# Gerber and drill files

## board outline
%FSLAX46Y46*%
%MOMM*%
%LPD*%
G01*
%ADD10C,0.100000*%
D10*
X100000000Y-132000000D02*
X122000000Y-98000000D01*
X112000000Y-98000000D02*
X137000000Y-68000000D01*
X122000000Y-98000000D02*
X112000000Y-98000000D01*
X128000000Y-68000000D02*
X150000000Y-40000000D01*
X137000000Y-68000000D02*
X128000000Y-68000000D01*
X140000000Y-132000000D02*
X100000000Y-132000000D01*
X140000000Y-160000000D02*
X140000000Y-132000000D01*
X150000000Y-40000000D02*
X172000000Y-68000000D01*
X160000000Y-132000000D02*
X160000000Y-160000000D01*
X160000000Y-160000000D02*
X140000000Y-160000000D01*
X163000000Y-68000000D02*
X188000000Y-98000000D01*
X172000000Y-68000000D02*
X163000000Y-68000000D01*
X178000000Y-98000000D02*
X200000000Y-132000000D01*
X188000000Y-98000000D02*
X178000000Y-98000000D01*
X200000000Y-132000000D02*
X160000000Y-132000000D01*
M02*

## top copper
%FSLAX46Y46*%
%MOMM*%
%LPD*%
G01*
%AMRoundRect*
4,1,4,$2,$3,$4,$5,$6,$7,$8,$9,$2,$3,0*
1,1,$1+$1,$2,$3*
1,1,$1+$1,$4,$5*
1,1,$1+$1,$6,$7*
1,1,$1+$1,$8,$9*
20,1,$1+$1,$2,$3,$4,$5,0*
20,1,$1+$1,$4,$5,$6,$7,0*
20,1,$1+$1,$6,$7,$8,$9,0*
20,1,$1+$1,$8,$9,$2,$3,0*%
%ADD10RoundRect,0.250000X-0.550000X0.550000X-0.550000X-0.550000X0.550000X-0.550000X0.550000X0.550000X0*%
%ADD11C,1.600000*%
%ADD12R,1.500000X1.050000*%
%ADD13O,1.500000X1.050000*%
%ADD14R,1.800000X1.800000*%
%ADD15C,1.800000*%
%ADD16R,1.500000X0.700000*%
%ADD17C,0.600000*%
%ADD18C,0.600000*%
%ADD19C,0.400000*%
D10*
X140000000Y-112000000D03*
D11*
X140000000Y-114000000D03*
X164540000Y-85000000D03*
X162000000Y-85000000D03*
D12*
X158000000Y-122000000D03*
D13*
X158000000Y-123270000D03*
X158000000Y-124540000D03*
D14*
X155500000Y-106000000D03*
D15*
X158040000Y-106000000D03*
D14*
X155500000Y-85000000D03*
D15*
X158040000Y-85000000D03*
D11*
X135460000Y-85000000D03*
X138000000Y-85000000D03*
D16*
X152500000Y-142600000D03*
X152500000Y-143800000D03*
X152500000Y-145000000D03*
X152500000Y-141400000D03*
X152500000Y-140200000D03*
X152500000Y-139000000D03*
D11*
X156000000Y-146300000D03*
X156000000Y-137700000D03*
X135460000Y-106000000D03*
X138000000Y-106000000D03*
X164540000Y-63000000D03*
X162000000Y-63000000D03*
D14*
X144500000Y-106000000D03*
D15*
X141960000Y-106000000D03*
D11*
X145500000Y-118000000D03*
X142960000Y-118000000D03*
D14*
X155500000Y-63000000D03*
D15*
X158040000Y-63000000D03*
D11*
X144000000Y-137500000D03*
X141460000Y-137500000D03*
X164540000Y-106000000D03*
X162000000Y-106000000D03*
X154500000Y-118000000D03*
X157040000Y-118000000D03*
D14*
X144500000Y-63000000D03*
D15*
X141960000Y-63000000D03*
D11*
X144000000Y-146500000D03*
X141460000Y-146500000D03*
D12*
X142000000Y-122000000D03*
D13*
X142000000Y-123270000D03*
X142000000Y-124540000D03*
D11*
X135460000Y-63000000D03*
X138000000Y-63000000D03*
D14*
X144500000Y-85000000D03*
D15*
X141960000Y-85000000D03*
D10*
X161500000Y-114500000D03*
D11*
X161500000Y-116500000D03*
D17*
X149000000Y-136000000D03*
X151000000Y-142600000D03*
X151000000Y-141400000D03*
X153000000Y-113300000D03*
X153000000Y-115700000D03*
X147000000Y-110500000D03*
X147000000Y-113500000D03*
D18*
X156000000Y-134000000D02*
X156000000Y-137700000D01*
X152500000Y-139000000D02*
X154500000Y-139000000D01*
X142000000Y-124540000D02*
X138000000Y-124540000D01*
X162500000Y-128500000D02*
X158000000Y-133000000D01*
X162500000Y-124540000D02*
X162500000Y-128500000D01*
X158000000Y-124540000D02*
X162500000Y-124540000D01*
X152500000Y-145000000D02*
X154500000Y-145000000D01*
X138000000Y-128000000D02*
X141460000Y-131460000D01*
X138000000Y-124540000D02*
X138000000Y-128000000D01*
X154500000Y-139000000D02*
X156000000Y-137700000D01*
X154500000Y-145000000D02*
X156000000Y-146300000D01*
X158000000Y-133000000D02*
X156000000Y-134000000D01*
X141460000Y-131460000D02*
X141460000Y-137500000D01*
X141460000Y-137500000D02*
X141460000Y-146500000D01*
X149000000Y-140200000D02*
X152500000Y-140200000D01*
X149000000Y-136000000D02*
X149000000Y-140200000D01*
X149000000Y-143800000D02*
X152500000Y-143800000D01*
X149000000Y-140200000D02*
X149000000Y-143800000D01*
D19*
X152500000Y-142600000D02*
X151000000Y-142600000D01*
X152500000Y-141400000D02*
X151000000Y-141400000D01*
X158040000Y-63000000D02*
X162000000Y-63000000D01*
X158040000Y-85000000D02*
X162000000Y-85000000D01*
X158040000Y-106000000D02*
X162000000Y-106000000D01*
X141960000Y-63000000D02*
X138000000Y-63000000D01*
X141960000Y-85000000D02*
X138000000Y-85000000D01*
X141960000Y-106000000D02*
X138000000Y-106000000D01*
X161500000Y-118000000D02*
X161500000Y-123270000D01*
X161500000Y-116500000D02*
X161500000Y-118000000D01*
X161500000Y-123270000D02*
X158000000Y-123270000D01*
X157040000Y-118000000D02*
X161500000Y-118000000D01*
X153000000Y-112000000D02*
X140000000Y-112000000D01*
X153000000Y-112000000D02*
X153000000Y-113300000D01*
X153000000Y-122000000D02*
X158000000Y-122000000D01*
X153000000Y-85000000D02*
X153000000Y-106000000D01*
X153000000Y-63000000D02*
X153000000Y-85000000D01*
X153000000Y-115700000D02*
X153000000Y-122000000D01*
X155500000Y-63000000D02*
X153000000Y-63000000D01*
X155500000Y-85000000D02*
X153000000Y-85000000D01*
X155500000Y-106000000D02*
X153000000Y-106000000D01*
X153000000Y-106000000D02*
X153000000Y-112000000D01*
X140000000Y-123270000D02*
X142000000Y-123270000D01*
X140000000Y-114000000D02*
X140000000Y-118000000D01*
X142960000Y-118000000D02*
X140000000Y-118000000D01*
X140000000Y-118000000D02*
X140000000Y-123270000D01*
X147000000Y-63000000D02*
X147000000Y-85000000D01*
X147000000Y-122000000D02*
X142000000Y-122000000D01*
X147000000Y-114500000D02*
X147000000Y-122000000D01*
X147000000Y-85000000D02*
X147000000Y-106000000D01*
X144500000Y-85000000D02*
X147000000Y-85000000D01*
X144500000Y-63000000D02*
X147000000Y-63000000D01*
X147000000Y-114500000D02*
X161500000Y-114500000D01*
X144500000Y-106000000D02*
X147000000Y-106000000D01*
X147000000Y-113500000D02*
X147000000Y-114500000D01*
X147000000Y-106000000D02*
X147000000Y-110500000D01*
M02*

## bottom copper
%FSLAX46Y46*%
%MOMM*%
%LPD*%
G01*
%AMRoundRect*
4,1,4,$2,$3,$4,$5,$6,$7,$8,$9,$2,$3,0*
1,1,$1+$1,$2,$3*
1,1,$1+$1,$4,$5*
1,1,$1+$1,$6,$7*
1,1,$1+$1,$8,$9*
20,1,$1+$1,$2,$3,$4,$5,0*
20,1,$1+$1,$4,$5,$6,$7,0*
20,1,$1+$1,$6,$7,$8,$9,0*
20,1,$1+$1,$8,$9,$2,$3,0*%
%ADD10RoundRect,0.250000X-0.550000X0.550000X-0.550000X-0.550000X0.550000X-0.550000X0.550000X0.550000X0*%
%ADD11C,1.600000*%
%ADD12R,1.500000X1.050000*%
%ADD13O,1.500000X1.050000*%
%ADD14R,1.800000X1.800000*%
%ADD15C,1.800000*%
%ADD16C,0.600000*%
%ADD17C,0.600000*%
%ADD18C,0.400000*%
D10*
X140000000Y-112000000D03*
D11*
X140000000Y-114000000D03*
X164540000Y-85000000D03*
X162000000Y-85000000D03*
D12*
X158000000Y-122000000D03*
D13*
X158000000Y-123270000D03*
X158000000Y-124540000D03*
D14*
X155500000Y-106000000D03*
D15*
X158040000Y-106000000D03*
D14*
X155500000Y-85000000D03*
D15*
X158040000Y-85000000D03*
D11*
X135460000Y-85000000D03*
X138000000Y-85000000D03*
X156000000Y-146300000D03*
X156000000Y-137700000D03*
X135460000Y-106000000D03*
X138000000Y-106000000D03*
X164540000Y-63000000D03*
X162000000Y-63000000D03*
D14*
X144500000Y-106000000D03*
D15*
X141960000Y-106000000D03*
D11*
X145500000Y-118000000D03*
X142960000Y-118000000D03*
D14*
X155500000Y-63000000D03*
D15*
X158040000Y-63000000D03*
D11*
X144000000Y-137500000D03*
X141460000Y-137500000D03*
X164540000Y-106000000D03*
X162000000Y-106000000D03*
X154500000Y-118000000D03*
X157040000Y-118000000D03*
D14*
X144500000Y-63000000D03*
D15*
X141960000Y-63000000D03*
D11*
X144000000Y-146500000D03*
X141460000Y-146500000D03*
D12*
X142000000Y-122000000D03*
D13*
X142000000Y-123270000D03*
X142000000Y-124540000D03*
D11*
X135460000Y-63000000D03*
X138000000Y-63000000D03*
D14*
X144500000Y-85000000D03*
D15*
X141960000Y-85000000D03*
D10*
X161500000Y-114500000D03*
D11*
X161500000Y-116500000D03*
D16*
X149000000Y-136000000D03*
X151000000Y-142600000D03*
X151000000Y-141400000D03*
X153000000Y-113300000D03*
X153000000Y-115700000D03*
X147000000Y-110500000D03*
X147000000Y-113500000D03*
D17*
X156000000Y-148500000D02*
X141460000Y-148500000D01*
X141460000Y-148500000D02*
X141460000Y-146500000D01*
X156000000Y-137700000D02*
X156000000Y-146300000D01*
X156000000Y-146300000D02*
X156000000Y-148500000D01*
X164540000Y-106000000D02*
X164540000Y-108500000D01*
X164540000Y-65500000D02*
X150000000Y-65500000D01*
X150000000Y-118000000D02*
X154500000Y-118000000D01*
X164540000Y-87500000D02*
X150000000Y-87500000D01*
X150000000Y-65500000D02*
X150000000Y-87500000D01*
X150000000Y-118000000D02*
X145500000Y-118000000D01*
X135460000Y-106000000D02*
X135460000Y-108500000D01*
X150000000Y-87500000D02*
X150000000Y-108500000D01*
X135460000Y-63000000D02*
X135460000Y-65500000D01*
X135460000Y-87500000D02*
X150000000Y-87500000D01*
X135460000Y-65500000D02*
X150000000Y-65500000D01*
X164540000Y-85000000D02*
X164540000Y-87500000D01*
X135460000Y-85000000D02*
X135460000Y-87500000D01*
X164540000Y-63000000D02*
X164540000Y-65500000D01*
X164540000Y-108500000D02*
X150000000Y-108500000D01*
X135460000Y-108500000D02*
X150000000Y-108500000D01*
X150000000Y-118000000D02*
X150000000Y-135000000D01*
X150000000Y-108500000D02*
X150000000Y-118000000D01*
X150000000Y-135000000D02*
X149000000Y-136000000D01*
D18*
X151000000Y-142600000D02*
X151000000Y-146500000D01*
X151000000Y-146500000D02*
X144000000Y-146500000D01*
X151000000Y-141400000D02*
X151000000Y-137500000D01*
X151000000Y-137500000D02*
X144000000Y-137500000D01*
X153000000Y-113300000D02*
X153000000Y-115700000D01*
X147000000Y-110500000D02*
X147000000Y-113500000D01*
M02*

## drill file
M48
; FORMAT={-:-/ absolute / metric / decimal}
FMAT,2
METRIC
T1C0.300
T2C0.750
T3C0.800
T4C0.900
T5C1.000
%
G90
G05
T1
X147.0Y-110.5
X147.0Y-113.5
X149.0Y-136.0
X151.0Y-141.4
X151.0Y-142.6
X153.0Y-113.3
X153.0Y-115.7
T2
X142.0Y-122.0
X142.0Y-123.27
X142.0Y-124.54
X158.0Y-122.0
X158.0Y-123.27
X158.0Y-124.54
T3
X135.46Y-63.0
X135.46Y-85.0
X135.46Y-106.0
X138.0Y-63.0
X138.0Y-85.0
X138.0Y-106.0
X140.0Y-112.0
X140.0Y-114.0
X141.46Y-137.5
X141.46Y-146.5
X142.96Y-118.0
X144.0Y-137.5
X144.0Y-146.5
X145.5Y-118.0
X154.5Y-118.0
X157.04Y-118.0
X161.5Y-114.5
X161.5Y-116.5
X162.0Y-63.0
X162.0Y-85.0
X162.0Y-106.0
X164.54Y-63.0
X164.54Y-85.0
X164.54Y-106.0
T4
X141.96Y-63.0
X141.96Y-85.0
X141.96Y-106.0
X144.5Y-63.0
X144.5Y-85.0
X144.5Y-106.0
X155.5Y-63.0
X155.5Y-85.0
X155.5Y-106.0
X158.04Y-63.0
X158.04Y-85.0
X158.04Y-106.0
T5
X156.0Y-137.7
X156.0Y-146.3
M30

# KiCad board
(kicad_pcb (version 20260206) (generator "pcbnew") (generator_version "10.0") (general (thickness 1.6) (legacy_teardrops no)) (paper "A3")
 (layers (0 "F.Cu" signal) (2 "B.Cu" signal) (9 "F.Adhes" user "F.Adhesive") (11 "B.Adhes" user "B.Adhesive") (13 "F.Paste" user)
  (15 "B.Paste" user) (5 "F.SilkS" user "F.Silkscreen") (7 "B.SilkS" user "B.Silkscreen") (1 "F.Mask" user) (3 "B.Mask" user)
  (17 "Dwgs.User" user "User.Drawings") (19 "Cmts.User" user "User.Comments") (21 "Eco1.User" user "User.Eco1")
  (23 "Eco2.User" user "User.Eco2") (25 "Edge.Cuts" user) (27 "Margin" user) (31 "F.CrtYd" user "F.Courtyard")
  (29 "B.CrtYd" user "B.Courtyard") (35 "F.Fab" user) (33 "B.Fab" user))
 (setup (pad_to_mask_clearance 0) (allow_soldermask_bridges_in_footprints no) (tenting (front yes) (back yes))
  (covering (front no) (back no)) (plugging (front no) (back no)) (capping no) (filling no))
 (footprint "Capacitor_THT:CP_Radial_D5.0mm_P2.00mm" (layer "F.Cu") (at 140 112 -90)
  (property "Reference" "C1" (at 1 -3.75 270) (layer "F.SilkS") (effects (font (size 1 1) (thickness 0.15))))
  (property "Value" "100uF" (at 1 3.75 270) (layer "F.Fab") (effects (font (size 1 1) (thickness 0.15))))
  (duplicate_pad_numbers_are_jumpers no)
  (pad "1" thru_hole roundrect (at 0 0 270) (size 1.6 1.6) (drill 0.8) (layers "*.Cu" "*.Mask") (remove_unused_layers no)
   (roundrect_rratio 0.15625) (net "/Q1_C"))
  (pad "2" thru_hole circle (at 2 0 270) (size 1.6 1.6) (drill 0.8) (layers "*.Cu" "*.Mask") (remove_unused_layers no) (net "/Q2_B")))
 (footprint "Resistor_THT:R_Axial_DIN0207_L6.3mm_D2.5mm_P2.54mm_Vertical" (layer "F.Cu") (at 164.54 85 180)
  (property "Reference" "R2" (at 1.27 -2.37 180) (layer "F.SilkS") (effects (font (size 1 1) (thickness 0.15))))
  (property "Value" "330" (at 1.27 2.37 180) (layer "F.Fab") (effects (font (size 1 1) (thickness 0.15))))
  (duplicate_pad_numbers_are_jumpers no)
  (pad "1" thru_hole circle (at 0 0 180) (size 1.6 1.6) (drill 0.8) (layers "*.Cu" "*.Mask") (remove_unused_layers no) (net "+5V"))
  (pad "2" thru_hole circle (at 2.54 0 180) (size 1.6 1.6) (drill 0.8) (layers "*.Cu" "*.Mask") (remove_unused_layers no) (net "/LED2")))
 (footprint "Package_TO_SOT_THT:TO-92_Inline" (layer "F.Cu") (at 158 122 -90)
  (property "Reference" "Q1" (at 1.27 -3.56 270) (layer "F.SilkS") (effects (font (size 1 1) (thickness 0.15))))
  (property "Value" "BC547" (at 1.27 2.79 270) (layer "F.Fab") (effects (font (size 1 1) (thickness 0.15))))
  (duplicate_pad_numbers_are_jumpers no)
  (pad "1" thru_hole rect (at 0 0 270) (size 1.05 1.5) (drill 0.75) (layers "*.Cu" "*.Mask") (remove_unused_layers no) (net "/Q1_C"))
  (pad "2" thru_hole oval (at 1.27 0 270) (size 1.05 1.5) (drill 0.75) (layers "*.Cu" "*.Mask") (remove_unused_layers no) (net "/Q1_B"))
  (pad "3" thru_hole oval (at 2.54 0 270) (size 1.05 1.5) (drill 0.75) (layers "*.Cu" "*.Mask") (remove_unused_layers no) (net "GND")))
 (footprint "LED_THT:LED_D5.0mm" (layer "F.Cu") (at 155.5 106)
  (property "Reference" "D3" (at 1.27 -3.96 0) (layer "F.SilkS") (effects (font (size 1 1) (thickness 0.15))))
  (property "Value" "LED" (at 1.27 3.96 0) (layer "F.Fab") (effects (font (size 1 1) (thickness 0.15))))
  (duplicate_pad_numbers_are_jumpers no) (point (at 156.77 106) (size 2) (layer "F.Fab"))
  (pad "1" thru_hole rect (at 0 0) (size 1.8 1.8) (drill 0.9) (layers "*.Cu" "*.Mask") (remove_unused_layers no) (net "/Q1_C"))
  (pad "2" thru_hole circle (at 2.54 0) (size 1.8 1.8) (drill 0.9) (layers "*.Cu" "*.Mask") (remove_unused_layers no) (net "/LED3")))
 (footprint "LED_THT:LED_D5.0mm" (layer "F.Cu") (at 155.5 85)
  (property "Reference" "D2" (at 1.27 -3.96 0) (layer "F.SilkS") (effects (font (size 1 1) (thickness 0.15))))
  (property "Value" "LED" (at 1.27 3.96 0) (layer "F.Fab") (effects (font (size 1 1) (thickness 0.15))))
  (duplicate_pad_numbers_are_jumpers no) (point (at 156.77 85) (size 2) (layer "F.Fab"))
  (pad "1" thru_hole rect (at 0 0) (size 1.8 1.8) (drill 0.9) (layers "*.Cu" "*.Mask") (remove_unused_layers no) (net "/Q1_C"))
  (pad "2" thru_hole circle (at 2.54 0) (size 1.8 1.8) (drill 0.9) (layers "*.Cu" "*.Mask") (remove_unused_layers no) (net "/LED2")))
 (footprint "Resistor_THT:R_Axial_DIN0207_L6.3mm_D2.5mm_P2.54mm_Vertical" (layer "F.Cu") (at 135.46 85)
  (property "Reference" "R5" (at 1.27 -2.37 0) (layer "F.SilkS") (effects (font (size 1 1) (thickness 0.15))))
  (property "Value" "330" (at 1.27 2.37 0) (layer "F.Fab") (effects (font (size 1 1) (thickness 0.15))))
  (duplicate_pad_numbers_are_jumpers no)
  (pad "1" thru_hole circle (at 0 0) (size 1.6 1.6) (drill 0.8) (layers "*.Cu" "*.Mask") (remove_unused_layers no) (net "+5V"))
  (pad "2" thru_hole circle (at 2.54 0) (size 1.6 1.6) (drill 0.8) (layers "*.Cu" "*.Mask") (remove_unused_layers no) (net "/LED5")))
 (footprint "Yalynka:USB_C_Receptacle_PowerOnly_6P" (layer "F.Cu") (at 152.5 142 90)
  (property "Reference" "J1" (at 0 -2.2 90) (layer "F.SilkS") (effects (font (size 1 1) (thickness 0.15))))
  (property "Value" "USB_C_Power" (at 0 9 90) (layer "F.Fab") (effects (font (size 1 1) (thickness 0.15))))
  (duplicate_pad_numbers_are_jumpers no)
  (pad "A5" smd rect (at -0.6 0 90) (size 0.7 1.5) (layers "F.Cu" "F.Mask" "F.Paste") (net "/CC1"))
  (pad "A9" smd rect (at -1.8 0 90) (size 0.7 1.5) (layers "F.Cu" "F.Mask" "F.Paste") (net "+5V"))
  (pad "A12" smd rect (at -3 0 90) (size 0.7 1.5) (layers "F.Cu" "F.Mask" "F.Paste") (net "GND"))
  (pad "B5" smd rect (at 0.6 0 90) (size 0.7 1.5) (layers "F.Cu" "F.Mask" "F.Paste") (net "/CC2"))
  (pad "B9" smd rect (at 1.8 0 90) (size 0.7 1.5) (layers "F.Cu" "F.Mask" "F.Paste") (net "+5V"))
  (pad "B12" smd rect (at 3 0 90) (size 0.7 1.5) (layers "F.Cu" "F.Mask" "F.Paste") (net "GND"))
  (pad "S1" thru_hole circle (at -4.3 3.5 90) (size 1.6 1.6) (drill 1) (layers "*.Cu" "*.Mask") (remove_unused_layers no) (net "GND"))
  (pad "S1" thru_hole circle (at 4.3 3.5 90) (size 1.6 1.6) (drill 1) (layers "*.Cu" "*.Mask") (remove_unused_layers no) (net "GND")))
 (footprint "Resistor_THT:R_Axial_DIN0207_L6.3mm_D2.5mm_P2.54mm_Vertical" (layer "F.Cu") (at 135.46 106)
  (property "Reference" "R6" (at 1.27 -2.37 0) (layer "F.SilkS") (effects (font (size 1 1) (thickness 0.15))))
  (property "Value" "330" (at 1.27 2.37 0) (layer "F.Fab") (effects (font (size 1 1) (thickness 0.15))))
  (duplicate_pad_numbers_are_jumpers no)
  (pad "1" thru_hole circle (at 0 0) (size 1.6 1.6) (drill 0.8) (layers "*.Cu" "*.Mask") (remove_unused_layers no) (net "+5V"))
  (pad "2" thru_hole circle (at 2.54 0) (size 1.6 1.6) (drill 0.8) (layers "*.Cu" "*.Mask") (remove_unused_layers no) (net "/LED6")))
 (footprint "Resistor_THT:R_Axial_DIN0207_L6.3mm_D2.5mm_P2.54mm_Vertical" (layer "F.Cu") (at 164.54 63 180)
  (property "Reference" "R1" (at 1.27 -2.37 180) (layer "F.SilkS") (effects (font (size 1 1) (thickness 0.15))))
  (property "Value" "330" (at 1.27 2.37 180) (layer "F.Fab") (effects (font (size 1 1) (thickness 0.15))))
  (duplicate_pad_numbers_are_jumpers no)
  (pad "1" thru_hole circle (at 0 0 180) (size 1.6 1.6) (drill 0.8) (layers "*.Cu" "*.Mask") (remove_unused_layers no) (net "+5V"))
  (pad "2" thru_hole circle (at 2.54 0 180) (size 1.6 1.6) (drill 0.8) (layers "*.Cu" "*.Mask") (remove_unused_layers no) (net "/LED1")))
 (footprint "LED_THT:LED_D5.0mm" (layer "F.Cu") (at 144.5 106 180)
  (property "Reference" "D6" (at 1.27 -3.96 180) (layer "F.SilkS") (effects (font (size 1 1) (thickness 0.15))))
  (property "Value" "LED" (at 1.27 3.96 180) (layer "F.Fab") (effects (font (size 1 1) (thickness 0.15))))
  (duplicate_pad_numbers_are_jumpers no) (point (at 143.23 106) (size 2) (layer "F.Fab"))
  (pad "1" thru_hole rect (at 0 0 180) (size 1.8 1.8) (drill 0.9) (layers "*.Cu" "*.Mask") (remove_unused_layers no) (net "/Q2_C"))
  (pad "2" thru_hole circle (at 2.54 0 180) (size 1.8 1.8) (drill 0.9) (layers "*.Cu" "*.Mask") (remove_unused_layers no) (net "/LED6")))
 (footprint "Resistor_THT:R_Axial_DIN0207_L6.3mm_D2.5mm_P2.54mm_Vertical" (layer "F.Cu") (at 145.5 118 180)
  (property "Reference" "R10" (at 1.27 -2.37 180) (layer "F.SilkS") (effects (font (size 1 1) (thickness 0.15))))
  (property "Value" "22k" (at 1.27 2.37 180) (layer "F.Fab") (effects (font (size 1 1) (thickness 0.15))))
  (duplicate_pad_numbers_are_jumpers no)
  (pad "1" thru_hole circle (at 0 0 180) (size 1.6 1.6) (drill 0.8) (layers "*.Cu" "*.Mask") (remove_unused_layers no) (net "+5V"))
  (pad "2" thru_hole circle (at 2.54 0 180) (size 1.6 1.6) (drill 0.8) (layers "*.Cu" "*.Mask") (remove_unused_layers no) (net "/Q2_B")))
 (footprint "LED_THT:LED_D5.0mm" (layer "F.Cu") (at 155.5 63)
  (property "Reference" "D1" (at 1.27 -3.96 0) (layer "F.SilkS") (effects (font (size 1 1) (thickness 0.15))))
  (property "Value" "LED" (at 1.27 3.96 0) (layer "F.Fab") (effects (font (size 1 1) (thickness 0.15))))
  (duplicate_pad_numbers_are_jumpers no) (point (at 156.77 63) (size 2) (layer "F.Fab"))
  (pad "1" thru_hole rect (at 0 0) (size 1.8 1.8) (drill 0.9) (layers "*.Cu" "*.Mask") (remove_unused_layers no) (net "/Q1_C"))
  (pad "2" thru_hole circle (at 2.54 0) (size 1.8 1.8) (drill 0.9) (layers "*.Cu" "*.Mask") (remove_unused_layers no) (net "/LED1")))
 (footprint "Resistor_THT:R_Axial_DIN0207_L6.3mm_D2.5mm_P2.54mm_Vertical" (layer "F.Cu") (at 144 137.5 180)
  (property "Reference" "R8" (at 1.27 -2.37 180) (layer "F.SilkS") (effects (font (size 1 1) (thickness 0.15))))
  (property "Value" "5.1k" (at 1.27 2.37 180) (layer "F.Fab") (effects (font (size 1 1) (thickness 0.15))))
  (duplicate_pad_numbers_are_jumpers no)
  (pad "1" thru_hole circle (at 0 0 180) (size 1.6 1.6) (drill 0.8) (layers "*.Cu" "*.Mask") (remove_unused_layers no) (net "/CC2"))
  (pad "2" thru_hole circle (at 2.54 0 180) (size 1.6 1.6) (drill 0.8) (layers "*.Cu" "*.Mask") (remove_unused_layers no) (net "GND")))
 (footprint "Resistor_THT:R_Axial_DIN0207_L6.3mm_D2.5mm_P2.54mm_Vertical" (layer "F.Cu") (at 164.54 106 180)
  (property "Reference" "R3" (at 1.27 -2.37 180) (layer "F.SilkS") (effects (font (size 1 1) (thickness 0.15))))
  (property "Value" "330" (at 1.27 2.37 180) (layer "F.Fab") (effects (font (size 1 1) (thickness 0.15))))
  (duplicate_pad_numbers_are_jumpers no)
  (pad "1" thru_hole circle (at 0 0 180) (size 1.6 1.6) (drill 0.8) (layers "*.Cu" "*.Mask") (remove_unused_layers no) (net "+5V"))
  (pad "2" thru_hole circle (at 2.54 0 180) (size 1.6 1.6) (drill 0.8) (layers "*.Cu" "*.Mask") (remove_unused_layers no) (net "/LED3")))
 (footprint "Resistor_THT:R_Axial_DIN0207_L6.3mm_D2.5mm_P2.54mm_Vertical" (layer "F.Cu") (at 154.5 118)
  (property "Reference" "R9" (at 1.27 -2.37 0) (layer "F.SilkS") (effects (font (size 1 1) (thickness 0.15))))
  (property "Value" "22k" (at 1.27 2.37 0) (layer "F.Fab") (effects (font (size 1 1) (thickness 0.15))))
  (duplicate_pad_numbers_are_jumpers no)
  (pad "1" thru_hole circle (at 0 0) (size 1.6 1.6) (drill 0.8) (layers "*.Cu" "*.Mask") (remove_unused_layers no) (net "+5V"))
  (pad "2" thru_hole circle (at 2.54 0) (size 1.6 1.6) (drill 0.8) (layers "*.Cu" "*.Mask") (remove_unused_layers no) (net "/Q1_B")))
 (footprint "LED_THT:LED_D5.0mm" (layer "F.Cu") (at 144.5 63 180)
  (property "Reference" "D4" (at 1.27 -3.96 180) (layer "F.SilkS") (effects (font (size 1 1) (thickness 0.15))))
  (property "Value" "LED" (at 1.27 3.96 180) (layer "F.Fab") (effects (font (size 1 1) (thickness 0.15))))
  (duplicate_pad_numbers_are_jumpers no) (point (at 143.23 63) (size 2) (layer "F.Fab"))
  (pad "1" thru_hole rect (at 0 0 180) (size 1.8 1.8) (drill 0.9) (layers "*.Cu" "*.Mask") (remove_unused_layers no) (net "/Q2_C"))
  (pad "2" thru_hole circle (at 2.54 0 180) (size 1.8 1.8) (drill 0.9) (layers "*.Cu" "*.Mask") (remove_unused_layers no) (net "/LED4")))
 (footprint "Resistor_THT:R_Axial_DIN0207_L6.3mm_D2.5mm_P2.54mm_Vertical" (layer "F.Cu") (at 144 146.5 180)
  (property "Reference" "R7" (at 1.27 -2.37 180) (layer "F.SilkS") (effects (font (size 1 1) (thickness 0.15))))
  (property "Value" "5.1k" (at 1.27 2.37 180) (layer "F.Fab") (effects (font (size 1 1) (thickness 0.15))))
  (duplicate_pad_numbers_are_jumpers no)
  (pad "1" thru_hole circle (at 0 0 180) (size 1.6 1.6) (drill 0.8) (layers "*.Cu" "*.Mask") (remove_unused_layers no) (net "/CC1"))
  (pad "2" thru_hole circle (at 2.54 0 180) (size 1.6 1.6) (drill 0.8) (layers "*.Cu" "*.Mask") (remove_unused_layers no) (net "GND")))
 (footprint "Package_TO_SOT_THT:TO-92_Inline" (layer "F.Cu") (at 142 122 -90)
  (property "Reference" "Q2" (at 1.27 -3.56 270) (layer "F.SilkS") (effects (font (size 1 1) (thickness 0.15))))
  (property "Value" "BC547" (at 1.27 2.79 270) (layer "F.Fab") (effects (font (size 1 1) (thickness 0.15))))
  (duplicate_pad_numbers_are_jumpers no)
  (pad "1" thru_hole rect (at 0 0 270) (size 1.05 1.5) (drill 0.75) (layers "*.Cu" "*.Mask") (remove_unused_layers no) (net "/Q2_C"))
  (pad "2" thru_hole oval (at 1.27 0 270) (size 1.05 1.5) (drill 0.75) (layers "*.Cu" "*.Mask") (remove_unused_layers no) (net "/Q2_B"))
  (pad "3" thru_hole oval (at 2.54 0 270) (size 1.05 1.5) (drill 0.75) (layers "*.Cu" "*.Mask") (remove_unused_layers no) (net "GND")))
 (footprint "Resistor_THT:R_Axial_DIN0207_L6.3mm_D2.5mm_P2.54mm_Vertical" (layer "F.Cu") (at 135.46 63)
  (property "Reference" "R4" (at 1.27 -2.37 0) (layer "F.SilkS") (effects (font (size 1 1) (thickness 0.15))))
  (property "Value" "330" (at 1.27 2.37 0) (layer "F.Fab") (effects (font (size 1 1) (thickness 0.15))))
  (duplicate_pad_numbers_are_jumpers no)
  (pad "1" thru_hole circle (at 0 0) (size 1.6 1.6) (drill 0.8) (layers "*.Cu" "*.Mask") (remove_unused_layers no) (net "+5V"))
  (pad "2" thru_hole circle (at 2.54 0) (size 1.6 1.6) (drill 0.8) (layers "*.Cu" "*.Mask") (remove_unused_layers no) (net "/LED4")))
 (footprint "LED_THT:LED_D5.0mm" (layer "F.Cu") (at 144.5 85 180)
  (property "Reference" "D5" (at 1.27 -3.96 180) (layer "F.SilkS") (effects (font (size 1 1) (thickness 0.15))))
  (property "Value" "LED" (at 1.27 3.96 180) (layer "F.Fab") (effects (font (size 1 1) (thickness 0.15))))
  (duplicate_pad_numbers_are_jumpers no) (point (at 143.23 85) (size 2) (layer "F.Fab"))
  (pad "1" thru_hole rect (at 0 0 180) (size 1.8 1.8) (drill 0.9) (layers "*.Cu" "*.Mask") (remove_unused_layers no) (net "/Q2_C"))
  (pad "2" thru_hole circle (at 2.54 0 180) (size 1.8 1.8) (drill 0.9) (layers "*.Cu" "*.Mask") (remove_unused_layers no) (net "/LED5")))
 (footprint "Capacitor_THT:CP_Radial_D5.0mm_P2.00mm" (layer "F.Cu") (at 161.5 114.5 -90)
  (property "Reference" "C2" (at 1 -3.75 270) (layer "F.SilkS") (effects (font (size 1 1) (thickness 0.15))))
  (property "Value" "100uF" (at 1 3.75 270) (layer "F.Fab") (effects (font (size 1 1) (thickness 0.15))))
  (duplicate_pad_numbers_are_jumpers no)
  (pad "1" thru_hole roundrect (at 0 0 270) (size 1.6 1.6) (drill 0.8) (layers "*.Cu" "*.Mask") (remove_unused_layers no)
   (roundrect_rratio 0.15625) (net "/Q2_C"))
  (pad "2" thru_hole circle (at 2 0 270) (size 1.6 1.6) (drill 0.8) (layers "*.Cu" "*.Mask") (remove_unused_layers no) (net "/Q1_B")))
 (gr_line (start 100 132) (end 122 98) (stroke (width 0.1) (type default)) (layer "Edge.Cuts"))
 (gr_line (start 112 98) (end 137 68) (stroke (width 0.1) (type default)) (layer "Edge.Cuts"))
 (gr_line (start 122 98) (end 112 98) (stroke (width 0.1) (type default)) (layer "Edge.Cuts"))
 (gr_line (start 128 68) (end 150 40) (stroke (width 0.1) (type default)) (layer "Edge.Cuts"))
 (gr_line (start 137 68) (end 128 68) (stroke (width 0.1) (type default)) (layer "Edge.Cuts"))
 (gr_line (start 140 132) (end 100 132) (stroke (width 0.1) (type default)) (layer "Edge.Cuts"))
 (gr_line (start 140 160) (end 140 132) (stroke (width 0.1) (type default)) (layer "Edge.Cuts"))
 (gr_line (start 150 40) (end 172 68) (stroke (width 0.1) (type default)) (layer "Edge.Cuts"))
 (gr_line (start 160 132) (end 160 160) (stroke (width 0.1) (type default)) (layer "Edge.Cuts"))
 (gr_line (start 160 160) (end 140 160) (stroke (width 0.1) (type default)) (layer "Edge.Cuts"))
 (gr_line (start 163 68) (end 188 98) (stroke (width 0.1) (type default)) (layer "Edge.Cuts"))
 (gr_line (start 172 68) (end 163 68) (stroke (width 0.1) (type default)) (layer "Edge.Cuts"))
 (gr_line (start 178 98) (end 200 132) (stroke (width 0.1) (type default)) (layer "Edge.Cuts"))
 (gr_line (start 188 98) (end 178 98) (stroke (width 0.1) (type default)) (layer "Edge.Cuts"))
 (gr_line (start 200 132) (end 160 132) (stroke (width 0.1) (type default)) (layer "Edge.Cuts"))
 (segment (start 156 134) (end 156 137.7) (width 0.6) (layer "F.Cu") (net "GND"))
 (segment (start 152.5 139) (end 154.5 139) (width 0.6) (layer "F.Cu") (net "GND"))
 (segment (start 142 124.54) (end 138 124.54) (width 0.6) (layer "F.Cu") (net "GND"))
 (segment (start 162.5 128.5) (end 158 133) (width 0.6) (layer "F.Cu") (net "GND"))
 (segment (start 162.5 124.54) (end 162.5 128.5) (width 0.6) (layer "F.Cu") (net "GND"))
 (segment (start 158 124.54) (end 162.5 124.54) (width 0.6) (layer "F.Cu") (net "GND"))
 (segment (start 152.5 145) (end 154.5 145) (width 0.6) (layer "F.Cu") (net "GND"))
 (segment (start 138 128) (end 141.46 131.46) (width 0.6) (layer "F.Cu") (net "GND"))
 (segment (start 138 124.54) (end 138 128) (width 0.6) (layer "F.Cu") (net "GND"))
 (segment (start 154.5 139) (end 156 137.7) (width 0.6) (layer "F.Cu") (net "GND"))
 (segment (start 154.5 145) (end 156 146.3) (width 0.6) (layer "F.Cu") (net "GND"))
 (segment (start 158 133) (end 156 134) (width 0.6) (layer "F.Cu") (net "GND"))
 (segment (start 141.46 131.46) (end 141.46 137.5) (width 0.6) (layer "F.Cu") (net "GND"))
 (segment (start 141.46 137.5) (end 141.46 146.5) (width 0.6) (layer "F.Cu") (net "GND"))
 (segment (start 156 148.5) (end 141.46 148.5) (width 0.6) (layer "B.Cu") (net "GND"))
 (segment (start 141.46 148.5) (end 141.46 146.5) (width 0.6) (layer "B.Cu") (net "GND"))
 (segment (start 156 137.7) (end 156 146.3) (width 0.6) (layer "B.Cu") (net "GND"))
 (segment (start 156 146.3) (end 156 148.5) (width 0.6) (layer "B.Cu") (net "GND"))
 (segment (start 149 140.2) (end 152.5 140.2) (width 0.6) (layer "F.Cu") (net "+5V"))
 (segment (start 149 136) (end 149 140.2) (width 0.6) (layer "F.Cu") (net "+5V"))
 (segment (start 149 143.8) (end 152.5 143.8) (width 0.6) (layer "F.Cu") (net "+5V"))
 (segment (start 149 140.2) (end 149 143.8) (width 0.6) (layer "F.Cu") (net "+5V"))
 (via (at 149 136) (size 0.6) (drill 0.3) (layers "F.Cu" "B.Cu") (capping no) (covering (front no) (back no))
  (plugging (front no) (back no)) (filling no) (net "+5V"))
 (segment (start 164.54 106) (end 164.54 108.5) (width 0.6) (layer "B.Cu") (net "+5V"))
 (segment (start 164.54 65.5) (end 150 65.5) (width 0.6) (layer "B.Cu") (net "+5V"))
 (segment (start 150 118) (end 154.5 118) (width 0.6) (layer "B.Cu") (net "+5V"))
 (segment (start 164.54 87.5) (end 150 87.5) (width 0.6) (layer "B.Cu") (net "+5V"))
 (segment (start 150 65.5) (end 150 87.5) (width 0.6) (layer "B.Cu") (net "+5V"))
 (segment (start 150 118) (end 145.5 118) (width 0.6) (layer "B.Cu") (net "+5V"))
 (segment (start 135.46 106) (end 135.46 108.5) (width 0.6) (layer "B.Cu") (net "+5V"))
 (segment (start 150 87.5) (end 150 108.5) (width 0.6) (layer "B.Cu") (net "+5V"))
 (segment (start 135.46 63) (end 135.46 65.5) (width 0.6) (layer "B.Cu") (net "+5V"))
 (segment (start 135.46 87.5) (end 150 87.5) (width 0.6) (layer "B.Cu") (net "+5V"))
 (segment (start 135.46 65.5) (end 150 65.5) (width 0.6) (layer "B.Cu") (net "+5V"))
 (segment (start 164.54 85) (end 164.54 87.5) (width 0.6) (layer "B.Cu") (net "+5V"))
 (segment (start 135.46 85) (end 135.46 87.5) (width 0.6) (layer "B.Cu") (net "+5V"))
 (segment (start 164.54 63) (end 164.54 65.5) (width 0.6) (layer "B.Cu") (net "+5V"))
 (segment (start 164.54 108.5) (end 150 108.5) (width 0.6) (layer "B.Cu") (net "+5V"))
 (segment (start 135.46 108.5) (end 150 108.5) (width 0.6) (layer "B.Cu") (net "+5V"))
 (segment (start 150 118) (end 150 135) (width 0.6) (layer "B.Cu") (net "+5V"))
 (segment (start 150 108.5) (end 150 118) (width 0.6) (layer "B.Cu") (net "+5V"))
 (segment (start 150 135) (end 149 136) (width 0.6) (layer "B.Cu") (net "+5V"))
 (segment (start 152.5 142.6) (end 151 142.6) (width 0.4) (layer "F.Cu") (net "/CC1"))
 (via (at 151 142.6) (size 0.6) (drill 0.3) (layers "F.Cu" "B.Cu") (capping no) (covering (front no) (back no))
  (plugging (front no) (back no)) (filling no) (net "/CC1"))
 (segment (start 151 142.6) (end 151 146.5) (width 0.4) (layer "B.Cu") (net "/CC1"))
 (segment (start 151 146.5) (end 144 146.5) (width 0.4) (layer "B.Cu") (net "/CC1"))
 (segment (start 152.5 141.4) (end 151 141.4) (width 0.4) (layer "F.Cu") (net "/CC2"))
 (via (at 151 141.4) (size 0.6) (drill 0.3) (layers "F.Cu" "B.Cu") (capping no) (covering (front no) (back no))
  (plugging (front no) (back no)) (filling no) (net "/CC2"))
 (segment (start 151 141.4) (end 151 137.5) (width 0.4) (layer "B.Cu") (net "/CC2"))
 (segment (start 151 137.5) (end 144 137.5) (width 0.4) (layer "B.Cu") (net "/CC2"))
 (segment (start 158.04 63) (end 162 63) (width 0.4) (layer "F.Cu") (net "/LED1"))
 (segment (start 158.04 85) (end 162 85) (width 0.4) (layer "F.Cu") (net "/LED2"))
 (segment (start 158.04 106) (end 162 106) (width 0.4) (layer "F.Cu") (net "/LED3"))
 (segment (start 141.96 63) (end 138 63) (width 0.4) (layer "F.Cu") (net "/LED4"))
 (segment (start 141.96 85) (end 138 85) (width 0.4) (layer "F.Cu") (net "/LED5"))
 (segment (start 141.96 106) (end 138 106) (width 0.4) (layer "F.Cu") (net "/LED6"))
 (segment (start 161.5 118) (end 161.5 123.27) (width 0.4) (layer "F.Cu") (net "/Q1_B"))
 (segment (start 161.5 116.5) (end 161.5 118) (width 0.4) (layer "F.Cu") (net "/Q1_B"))
 (segment (start 161.5 123.27) (end 158 123.27) (width 0.4) (layer "F.Cu") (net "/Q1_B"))
 (segment (start 157.04 118) (end 161.5 118) (width 0.4) (layer "F.Cu") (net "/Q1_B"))
 (segment (start 153 112) (end 140 112) (width 0.4) (layer "F.Cu") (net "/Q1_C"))
 (segment (start 153 112) (end 153 113.3) (width 0.4) (layer "F.Cu") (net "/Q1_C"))
 (segment (start 153 122) (end 158 122) (width 0.4) (layer "F.Cu") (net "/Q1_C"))
 (segment (start 153 85) (end 153 106) (width 0.4) (layer "F.Cu") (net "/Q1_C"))
 (segment (start 153 63) (end 153 85) (width 0.4) (layer "F.Cu") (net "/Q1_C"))
 (segment (start 153 115.7) (end 153 122) (width 0.4) (layer "F.Cu") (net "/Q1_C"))
 (segment (start 155.5 63) (end 153 63) (width 0.4) (layer "F.Cu") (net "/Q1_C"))
 (segment (start 155.5 85) (end 153 85) (width 0.4) (layer "F.Cu") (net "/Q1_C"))
 (segment (start 155.5 106) (end 153 106) (width 0.4) (layer "F.Cu") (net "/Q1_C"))
 (segment (start 153 106) (end 153 112) (width 0.4) (layer "F.Cu") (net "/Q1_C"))
 (via (at 153 113.3) (size 0.6) (drill 0.3) (layers "F.Cu" "B.Cu") (capping no) (covering (front no) (back no))
  (plugging (front no) (back no)) (filling no) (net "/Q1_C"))
 (via (at 153 115.7) (size 0.6) (drill 0.3) (layers "F.Cu" "B.Cu") (capping no) (covering (front no) (back no))
  (plugging (front no) (back no)) (filling no) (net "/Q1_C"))
 (segment (start 153 113.3) (end 153 115.7) (width 0.4) (layer "B.Cu") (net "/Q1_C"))
 (segment (start 140 123.27) (end 142 123.27) (width 0.4) (layer "F.Cu") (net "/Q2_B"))
 (segment (start 140 114) (end 140 118) (width 0.4) (layer "F.Cu") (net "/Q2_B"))
 (segment (start 142.96 118) (end 140 118) (width 0.4) (layer "F.Cu") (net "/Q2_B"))
 (segment (start 140 118) (end 140 123.27) (width 0.4) (layer "F.Cu") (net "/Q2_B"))
 (segment (start 147 63) (end 147 85) (width 0.4) (layer "F.Cu") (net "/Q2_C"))
 (segment (start 147 122) (end 142 122) (width 0.4) (layer "F.Cu") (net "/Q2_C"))
 (segment (start 147 114.5) (end 147 122) (width 0.4) (layer "F.Cu") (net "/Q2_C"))
 (segment (start 147 85) (end 147 106) (width 0.4) (layer "F.Cu") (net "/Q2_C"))
 (segment (start 144.5 85) (end 147 85) (width 0.4) (layer "F.Cu") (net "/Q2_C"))
 (segment (start 144.5 63) (end 147 63) (width 0.4) (layer "F.Cu") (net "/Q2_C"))
 (segment (start 147 114.5) (end 161.5 114.5) (width 0.4) (layer "F.Cu") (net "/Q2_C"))
 (segment (start 144.5 106) (end 147 106) (width 0.4) (layer "F.Cu") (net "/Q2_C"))
 (segment (start 147 113.5) (end 147 114.5) (width 0.4) (layer "F.Cu") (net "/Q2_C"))
 (segment (start 147 106) (end 147 110.5) (width 0.4) (layer "F.Cu") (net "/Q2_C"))
 (via (at 147 110.5) (size 0.6) (drill 0.3) (layers "F.Cu" "B.Cu") (capping no) (covering (front no) (back no))
  (plugging (front no) (back no)) (filling no) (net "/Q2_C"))
 (via (at 147 113.5) (size 0.6) (drill 0.3) (layers "F.Cu" "B.Cu") (capping no) (covering (front no) (back no))
  (plugging (front no) (back no)) (filling no) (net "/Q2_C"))
 (segment (start 147 110.5) (end 147 113.5) (width 0.4) (layer "B.Cu") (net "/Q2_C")))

